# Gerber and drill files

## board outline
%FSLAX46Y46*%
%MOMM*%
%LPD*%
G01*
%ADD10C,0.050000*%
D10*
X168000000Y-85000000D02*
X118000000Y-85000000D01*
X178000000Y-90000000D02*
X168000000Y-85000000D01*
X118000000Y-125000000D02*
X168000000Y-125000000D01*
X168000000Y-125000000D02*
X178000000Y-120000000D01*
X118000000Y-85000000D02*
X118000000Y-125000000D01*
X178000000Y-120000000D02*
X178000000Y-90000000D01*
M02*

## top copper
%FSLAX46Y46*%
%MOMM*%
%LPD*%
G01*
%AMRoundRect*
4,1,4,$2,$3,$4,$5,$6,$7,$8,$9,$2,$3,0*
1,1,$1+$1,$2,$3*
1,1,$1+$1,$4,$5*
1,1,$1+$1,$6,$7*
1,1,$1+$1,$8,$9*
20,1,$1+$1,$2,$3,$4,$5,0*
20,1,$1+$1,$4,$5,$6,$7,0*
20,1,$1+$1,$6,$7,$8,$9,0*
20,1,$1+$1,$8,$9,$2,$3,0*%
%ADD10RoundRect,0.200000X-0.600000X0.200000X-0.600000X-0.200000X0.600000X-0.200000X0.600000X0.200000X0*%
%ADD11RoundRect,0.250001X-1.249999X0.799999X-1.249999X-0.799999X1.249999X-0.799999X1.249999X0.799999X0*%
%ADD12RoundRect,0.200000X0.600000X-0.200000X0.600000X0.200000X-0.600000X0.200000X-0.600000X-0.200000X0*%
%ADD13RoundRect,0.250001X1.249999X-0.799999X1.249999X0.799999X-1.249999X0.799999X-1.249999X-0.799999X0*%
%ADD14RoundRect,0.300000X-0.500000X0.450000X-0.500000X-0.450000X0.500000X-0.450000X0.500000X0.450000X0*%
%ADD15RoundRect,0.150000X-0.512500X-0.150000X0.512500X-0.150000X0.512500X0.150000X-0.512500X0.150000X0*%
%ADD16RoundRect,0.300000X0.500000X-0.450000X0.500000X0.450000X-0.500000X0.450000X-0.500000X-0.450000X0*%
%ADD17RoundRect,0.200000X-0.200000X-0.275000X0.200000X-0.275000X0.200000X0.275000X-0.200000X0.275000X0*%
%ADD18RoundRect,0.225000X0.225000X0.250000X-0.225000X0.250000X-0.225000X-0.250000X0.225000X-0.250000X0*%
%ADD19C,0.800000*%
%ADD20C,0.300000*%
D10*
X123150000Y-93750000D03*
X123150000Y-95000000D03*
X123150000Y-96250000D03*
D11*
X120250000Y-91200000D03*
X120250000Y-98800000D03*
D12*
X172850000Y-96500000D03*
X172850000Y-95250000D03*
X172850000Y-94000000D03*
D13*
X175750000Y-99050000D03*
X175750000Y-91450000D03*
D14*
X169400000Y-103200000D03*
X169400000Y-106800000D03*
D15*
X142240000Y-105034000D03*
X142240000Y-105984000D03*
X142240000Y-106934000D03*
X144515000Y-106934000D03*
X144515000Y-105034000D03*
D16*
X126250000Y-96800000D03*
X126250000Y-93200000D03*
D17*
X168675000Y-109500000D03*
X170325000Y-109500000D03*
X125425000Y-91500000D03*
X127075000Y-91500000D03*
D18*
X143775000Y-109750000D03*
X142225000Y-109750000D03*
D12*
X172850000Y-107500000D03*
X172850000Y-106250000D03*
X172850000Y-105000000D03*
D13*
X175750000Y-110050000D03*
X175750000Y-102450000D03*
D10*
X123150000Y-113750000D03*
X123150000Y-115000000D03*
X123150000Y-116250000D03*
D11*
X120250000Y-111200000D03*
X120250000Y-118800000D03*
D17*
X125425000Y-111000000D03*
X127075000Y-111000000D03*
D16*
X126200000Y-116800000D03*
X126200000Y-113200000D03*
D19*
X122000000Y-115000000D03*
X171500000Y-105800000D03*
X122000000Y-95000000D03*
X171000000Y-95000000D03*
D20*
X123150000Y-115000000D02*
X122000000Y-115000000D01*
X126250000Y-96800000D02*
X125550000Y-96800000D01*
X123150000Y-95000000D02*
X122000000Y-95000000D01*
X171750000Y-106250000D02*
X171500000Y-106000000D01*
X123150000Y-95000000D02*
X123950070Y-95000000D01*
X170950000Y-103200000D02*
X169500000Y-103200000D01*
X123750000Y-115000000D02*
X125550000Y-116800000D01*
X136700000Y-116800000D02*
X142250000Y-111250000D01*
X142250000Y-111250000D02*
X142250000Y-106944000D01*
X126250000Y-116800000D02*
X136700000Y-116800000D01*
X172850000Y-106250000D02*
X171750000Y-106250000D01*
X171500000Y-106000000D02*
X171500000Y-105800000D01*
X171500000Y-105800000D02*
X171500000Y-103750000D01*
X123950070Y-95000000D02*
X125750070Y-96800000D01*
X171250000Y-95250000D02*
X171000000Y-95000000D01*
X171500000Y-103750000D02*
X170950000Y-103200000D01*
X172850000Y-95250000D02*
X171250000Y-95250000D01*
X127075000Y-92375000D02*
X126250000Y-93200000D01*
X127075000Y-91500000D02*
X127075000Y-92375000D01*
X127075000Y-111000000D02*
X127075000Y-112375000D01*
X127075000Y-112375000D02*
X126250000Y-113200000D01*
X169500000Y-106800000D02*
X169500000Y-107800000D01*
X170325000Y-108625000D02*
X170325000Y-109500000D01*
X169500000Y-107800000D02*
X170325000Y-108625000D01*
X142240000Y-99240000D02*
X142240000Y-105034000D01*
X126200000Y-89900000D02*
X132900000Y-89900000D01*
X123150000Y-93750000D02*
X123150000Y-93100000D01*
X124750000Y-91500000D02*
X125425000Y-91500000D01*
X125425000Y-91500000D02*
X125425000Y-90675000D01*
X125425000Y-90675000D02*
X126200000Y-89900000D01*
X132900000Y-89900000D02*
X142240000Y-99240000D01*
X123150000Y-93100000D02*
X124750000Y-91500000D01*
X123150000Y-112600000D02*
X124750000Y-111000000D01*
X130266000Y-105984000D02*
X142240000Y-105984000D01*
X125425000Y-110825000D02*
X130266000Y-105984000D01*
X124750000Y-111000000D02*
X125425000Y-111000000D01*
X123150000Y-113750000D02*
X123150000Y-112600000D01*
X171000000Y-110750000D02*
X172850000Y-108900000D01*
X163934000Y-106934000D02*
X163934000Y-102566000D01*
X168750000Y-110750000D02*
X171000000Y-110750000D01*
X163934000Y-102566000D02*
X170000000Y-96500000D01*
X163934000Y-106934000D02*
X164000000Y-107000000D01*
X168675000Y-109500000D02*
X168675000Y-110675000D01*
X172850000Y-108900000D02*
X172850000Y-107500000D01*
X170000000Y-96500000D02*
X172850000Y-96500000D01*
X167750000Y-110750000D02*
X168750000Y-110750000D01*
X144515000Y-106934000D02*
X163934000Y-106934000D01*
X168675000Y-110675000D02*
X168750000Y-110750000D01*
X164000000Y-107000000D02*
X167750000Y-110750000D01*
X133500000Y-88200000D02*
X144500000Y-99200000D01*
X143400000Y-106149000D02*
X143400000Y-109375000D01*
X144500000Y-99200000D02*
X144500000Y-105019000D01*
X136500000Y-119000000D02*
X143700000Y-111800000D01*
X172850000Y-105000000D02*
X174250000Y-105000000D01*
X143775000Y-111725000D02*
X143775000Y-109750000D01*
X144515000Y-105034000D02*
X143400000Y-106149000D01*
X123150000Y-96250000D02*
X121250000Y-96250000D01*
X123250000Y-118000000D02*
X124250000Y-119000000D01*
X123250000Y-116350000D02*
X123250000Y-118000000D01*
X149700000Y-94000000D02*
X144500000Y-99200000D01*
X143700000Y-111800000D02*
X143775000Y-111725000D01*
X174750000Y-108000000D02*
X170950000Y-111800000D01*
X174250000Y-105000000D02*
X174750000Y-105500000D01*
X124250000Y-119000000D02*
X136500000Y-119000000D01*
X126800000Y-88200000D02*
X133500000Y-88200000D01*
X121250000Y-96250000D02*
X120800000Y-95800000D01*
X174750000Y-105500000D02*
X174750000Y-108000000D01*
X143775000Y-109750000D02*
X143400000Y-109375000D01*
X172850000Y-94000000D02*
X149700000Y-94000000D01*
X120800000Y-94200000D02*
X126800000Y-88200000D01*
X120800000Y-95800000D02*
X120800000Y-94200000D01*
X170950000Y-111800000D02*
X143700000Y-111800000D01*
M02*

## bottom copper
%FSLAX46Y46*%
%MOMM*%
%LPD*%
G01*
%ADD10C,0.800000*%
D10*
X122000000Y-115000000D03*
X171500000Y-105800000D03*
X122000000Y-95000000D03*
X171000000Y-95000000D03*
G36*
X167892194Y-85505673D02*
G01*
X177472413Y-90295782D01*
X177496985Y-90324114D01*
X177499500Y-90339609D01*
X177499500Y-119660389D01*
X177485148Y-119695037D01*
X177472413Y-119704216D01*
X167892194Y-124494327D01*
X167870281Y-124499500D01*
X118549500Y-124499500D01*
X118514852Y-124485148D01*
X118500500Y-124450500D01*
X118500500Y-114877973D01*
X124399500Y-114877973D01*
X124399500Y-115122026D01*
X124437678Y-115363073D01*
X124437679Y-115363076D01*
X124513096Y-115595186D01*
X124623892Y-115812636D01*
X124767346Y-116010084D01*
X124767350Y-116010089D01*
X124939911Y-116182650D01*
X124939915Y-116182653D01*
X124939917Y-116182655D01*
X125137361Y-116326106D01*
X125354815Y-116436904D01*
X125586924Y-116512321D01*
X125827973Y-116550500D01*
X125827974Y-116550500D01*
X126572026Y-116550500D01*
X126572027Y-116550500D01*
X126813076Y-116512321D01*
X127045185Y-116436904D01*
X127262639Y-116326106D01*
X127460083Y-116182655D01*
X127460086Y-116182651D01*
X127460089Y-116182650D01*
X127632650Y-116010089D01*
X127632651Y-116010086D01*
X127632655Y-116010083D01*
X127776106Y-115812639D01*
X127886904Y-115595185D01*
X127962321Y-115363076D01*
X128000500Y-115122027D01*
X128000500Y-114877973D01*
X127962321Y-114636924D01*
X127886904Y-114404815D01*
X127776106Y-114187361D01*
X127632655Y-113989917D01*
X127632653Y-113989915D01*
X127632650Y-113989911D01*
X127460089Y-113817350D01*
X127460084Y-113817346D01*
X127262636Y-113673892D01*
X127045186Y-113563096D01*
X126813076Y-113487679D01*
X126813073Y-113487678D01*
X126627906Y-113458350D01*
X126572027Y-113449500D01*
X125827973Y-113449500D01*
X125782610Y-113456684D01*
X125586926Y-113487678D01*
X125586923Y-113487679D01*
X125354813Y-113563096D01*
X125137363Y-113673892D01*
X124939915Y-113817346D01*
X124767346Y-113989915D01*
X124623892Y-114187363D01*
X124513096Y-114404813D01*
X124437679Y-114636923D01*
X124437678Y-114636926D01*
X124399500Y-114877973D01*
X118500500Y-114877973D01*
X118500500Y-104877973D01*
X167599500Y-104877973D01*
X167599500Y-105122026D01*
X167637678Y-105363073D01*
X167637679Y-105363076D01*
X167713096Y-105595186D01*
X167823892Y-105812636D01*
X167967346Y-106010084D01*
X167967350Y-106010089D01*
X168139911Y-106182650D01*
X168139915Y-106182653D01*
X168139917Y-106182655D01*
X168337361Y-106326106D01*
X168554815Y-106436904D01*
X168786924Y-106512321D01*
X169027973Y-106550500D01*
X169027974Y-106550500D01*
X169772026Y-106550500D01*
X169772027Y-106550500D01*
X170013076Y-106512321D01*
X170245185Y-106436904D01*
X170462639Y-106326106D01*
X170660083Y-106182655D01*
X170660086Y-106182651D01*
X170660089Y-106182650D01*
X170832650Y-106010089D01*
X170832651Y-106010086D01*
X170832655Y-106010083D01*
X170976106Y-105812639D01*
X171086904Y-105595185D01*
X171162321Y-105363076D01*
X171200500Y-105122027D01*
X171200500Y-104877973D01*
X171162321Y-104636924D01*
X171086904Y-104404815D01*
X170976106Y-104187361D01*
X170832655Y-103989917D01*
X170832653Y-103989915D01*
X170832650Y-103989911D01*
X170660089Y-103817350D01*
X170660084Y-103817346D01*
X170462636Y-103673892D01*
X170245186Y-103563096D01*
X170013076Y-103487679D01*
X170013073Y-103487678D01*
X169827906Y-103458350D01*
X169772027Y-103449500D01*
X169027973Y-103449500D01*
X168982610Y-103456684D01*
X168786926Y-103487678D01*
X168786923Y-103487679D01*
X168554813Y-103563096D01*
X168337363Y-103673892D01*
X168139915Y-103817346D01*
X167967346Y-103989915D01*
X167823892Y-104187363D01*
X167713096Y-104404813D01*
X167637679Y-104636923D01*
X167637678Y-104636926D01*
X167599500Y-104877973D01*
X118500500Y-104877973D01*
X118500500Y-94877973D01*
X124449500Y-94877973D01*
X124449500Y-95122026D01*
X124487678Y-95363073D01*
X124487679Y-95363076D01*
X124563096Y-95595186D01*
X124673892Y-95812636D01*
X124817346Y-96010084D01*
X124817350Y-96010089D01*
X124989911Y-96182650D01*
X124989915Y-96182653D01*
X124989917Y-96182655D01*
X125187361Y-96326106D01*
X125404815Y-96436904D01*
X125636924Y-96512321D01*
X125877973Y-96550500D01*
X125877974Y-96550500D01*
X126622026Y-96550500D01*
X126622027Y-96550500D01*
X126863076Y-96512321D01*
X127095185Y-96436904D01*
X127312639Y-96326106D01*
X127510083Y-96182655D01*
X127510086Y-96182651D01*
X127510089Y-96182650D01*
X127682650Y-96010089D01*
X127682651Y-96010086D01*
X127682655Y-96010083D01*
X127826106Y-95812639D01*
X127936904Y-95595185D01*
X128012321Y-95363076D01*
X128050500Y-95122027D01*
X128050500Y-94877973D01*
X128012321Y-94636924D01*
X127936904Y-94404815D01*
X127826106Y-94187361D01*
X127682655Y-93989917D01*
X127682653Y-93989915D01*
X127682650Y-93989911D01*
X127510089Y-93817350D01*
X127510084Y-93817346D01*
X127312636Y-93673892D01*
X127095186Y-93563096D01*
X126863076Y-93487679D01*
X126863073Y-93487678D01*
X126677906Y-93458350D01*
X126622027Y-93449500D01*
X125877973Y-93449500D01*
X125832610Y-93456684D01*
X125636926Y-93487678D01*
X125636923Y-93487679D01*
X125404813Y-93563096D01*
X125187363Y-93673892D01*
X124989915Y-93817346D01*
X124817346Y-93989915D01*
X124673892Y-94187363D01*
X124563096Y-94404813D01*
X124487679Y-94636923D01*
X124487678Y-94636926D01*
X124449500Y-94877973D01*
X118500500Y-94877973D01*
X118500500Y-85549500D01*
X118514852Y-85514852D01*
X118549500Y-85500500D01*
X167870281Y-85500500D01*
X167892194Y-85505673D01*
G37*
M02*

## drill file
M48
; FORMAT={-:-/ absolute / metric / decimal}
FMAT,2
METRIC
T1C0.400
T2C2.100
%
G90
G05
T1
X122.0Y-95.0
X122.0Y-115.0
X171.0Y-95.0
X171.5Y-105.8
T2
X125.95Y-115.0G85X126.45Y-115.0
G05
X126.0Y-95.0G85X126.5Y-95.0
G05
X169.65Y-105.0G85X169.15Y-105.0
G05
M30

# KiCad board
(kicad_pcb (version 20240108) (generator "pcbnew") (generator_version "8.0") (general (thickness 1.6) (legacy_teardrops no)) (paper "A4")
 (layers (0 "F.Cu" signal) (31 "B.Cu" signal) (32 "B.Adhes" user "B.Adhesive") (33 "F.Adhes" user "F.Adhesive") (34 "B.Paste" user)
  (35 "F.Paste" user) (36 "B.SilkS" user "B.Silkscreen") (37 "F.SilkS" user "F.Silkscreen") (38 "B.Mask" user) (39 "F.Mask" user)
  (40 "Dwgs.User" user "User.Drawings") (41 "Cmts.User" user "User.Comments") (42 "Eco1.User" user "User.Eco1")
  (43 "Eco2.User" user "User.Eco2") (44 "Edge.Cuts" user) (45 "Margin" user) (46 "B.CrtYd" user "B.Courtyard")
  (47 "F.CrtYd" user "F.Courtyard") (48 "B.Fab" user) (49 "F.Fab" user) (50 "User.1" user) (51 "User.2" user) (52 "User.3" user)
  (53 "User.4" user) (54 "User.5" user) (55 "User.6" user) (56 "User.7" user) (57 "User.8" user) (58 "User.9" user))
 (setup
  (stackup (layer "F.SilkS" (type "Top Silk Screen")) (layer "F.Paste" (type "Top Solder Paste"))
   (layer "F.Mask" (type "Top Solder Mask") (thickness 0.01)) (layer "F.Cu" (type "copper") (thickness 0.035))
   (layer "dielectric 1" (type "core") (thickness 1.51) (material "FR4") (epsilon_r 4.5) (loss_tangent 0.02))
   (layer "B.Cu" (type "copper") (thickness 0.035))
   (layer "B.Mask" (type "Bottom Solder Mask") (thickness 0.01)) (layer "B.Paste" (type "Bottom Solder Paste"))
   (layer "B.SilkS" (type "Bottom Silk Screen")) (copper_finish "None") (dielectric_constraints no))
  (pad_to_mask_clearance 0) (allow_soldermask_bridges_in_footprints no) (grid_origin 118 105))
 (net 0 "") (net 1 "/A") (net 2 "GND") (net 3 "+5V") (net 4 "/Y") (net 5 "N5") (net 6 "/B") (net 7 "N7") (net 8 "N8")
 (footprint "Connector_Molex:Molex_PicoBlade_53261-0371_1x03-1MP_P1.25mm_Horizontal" (layer "F.Cu") (at 120.75 95 -90)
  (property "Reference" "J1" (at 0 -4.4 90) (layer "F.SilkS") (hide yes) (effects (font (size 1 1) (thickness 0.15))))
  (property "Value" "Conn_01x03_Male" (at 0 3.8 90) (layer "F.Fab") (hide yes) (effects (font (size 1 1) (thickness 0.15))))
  (pad "1" smd roundrect (at -1.25 -2.4 270) (size 0.8 1.6) (layers "F.Cu" "F.Paste" "F.Mask") (roundrect_rratio 0.25) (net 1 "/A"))
  (pad "2" smd roundrect (at 0 -2.4 270) (size 0.8 1.6) (layers "F.Cu" "F.Paste" "F.Mask") (roundrect_rratio 0.25) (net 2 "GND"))
  (pad "3" smd roundrect (at 1.25 -2.4 270) (size 0.8 1.6) (layers "F.Cu" "F.Paste" "F.Mask") (roundrect_rratio 0.25) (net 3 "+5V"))
  (pad "MP" smd roundrect (at -3.8 0.5 270) (size 2.1 3) (layers "F.Cu" "F.Paste" "F.Mask") (roundrect_rratio 0.1190480952))
  (pad "MP" smd roundrect (at 3.8 0.5 270) (size 2.1 3) (layers "F.Cu" "F.Paste" "F.Mask") (roundrect_rratio 0.1190480952)))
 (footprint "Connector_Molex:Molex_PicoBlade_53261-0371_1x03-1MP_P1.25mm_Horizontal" (layer "F.Cu") (at 175.25 95.25 90)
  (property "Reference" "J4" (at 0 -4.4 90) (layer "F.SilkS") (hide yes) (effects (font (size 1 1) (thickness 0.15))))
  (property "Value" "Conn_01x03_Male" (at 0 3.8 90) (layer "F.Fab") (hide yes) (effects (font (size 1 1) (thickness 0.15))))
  (pad "1" smd roundrect (at -1.25 -2.4 90) (size 0.8 1.6) (layers "F.Cu" "F.Paste" "F.Mask") (roundrect_rratio 0.25) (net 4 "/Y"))
  (pad "2" smd roundrect (at 0 -2.4 90) (size 0.8 1.6) (layers "F.Cu" "F.Paste" "F.Mask") (roundrect_rratio 0.25) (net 2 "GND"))
  (pad "3" smd roundrect (at 1.25 -2.4 90) (size 0.8 1.6) (layers "F.Cu" "F.Paste" "F.Mask") (roundrect_rratio 0.25) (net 3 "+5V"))
  (pad "MP" smd roundrect (at -3.8 0.5 90) (size 2.1 3) (layers "F.Cu" "F.Paste" "F.Mask") (roundrect_rratio 0.1190480952))
  (pad "MP" smd roundrect (at 3.8 0.5 90) (size 2.1 3) (layers "F.Cu" "F.Paste" "F.Mask") (roundrect_rratio 0.1190480952)))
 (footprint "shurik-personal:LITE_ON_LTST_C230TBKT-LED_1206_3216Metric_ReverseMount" (layer "F.Cu") (at 169.4 105 -90)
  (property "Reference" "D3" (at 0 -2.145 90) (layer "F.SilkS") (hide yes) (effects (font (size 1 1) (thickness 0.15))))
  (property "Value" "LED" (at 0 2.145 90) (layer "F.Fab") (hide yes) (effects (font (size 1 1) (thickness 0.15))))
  (pad "" np_thru_hole oval (at 0 0 270) (size 2.1 2.6) (drill oval 2.1 2.6) (layers "F&B.Cu" "*.Mask"))
  (pad "1" smd roundrect (at -1.8 0 270) (size 1.5 1.6) (layers "F.Cu" "F.Paste" "F.Mask") (roundrect_rratio 0.2) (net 2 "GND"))
  (pad "2" smd roundrect (at 1.8 0 270) (size 1.5 1.6) (layers "F.Cu" "F.Paste" "F.Mask") (roundrect_rratio 0.2) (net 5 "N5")))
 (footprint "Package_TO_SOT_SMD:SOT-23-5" (layer "F.Cu") (at 143.3775 105.984)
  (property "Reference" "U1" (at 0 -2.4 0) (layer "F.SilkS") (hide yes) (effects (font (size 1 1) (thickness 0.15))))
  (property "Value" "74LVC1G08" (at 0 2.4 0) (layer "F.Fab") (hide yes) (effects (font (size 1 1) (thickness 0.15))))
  (pad "1" smd roundrect (at -1.1375 -0.95) (size 1.325 0.6) (layers "F.Cu" "F.Paste" "F.Mask") (roundrect_rratio 0.25) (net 1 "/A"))
  (pad "2" smd roundrect (at -1.1375 0) (size 1.325 0.6) (layers "F.Cu" "F.Paste" "F.Mask") (roundrect_rratio 0.25) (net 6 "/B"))
  (pad "3" smd roundrect (at -1.1375 0.95) (size 1.325 0.6) (layers "F.Cu" "F.Paste" "F.Mask") (roundrect_rratio 0.25) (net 2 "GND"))
  (pad "4" smd roundrect (at 1.1375 0.95) (size 1.325 0.6) (layers "F.Cu" "F.Paste" "F.Mask") (roundrect_rratio 0.25) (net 4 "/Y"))
  (pad "5" smd roundrect (at 1.1375 -0.95) (size 1.325 0.6) (layers "F.Cu" "F.Paste" "F.Mask") (roundrect_rratio 0.25) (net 3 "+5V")))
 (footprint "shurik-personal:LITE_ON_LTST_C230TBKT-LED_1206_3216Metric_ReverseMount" (layer "F.Cu") (at 126.25 95 90)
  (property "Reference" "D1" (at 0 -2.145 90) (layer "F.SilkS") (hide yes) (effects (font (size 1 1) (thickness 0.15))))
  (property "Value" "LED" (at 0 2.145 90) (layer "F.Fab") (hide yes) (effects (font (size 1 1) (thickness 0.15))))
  (pad "" np_thru_hole oval (at 0 0 90) (size 2.1 2.6) (drill oval 2.1 2.6) (layers "F&B.Cu" "*.Mask"))
  (pad "1" smd roundrect (at -1.8 0 90) (size 1.5 1.6) (layers "F.Cu" "F.Paste" "F.Mask") (roundrect_rratio 0.2) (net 2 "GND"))
  (pad "2" smd roundrect (at 1.8 0 90) (size 1.5 1.6) (layers "F.Cu" "F.Paste" "F.Mask") (roundrect_rratio 0.2) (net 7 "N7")))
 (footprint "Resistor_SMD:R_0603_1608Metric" (layer "F.Cu") (at 169.5 109.5)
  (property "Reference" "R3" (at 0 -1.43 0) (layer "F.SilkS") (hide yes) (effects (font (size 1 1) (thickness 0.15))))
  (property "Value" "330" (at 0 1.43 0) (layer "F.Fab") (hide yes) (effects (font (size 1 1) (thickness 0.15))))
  (pad "1" smd roundrect (at -0.825 0) (size 0.8 0.95) (layers "F.Cu" "F.Paste" "F.Mask") (roundrect_rratio 0.25) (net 4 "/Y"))
  (pad "2" smd roundrect (at 0.825 0) (size 0.8 0.95) (layers "F.Cu" "F.Paste" "F.Mask") (roundrect_rratio 0.25) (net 5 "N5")))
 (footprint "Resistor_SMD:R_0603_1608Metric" (layer "F.Cu") (at 126.25 91.5)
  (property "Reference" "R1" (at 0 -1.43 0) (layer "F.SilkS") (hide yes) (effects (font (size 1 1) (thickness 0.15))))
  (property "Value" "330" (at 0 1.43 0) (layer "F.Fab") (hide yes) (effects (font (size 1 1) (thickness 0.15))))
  (pad "1" smd roundrect (at -0.825 0) (size 0.8 0.95) (layers "F.Cu" "F.Paste" "F.Mask") (roundrect_rratio 0.25) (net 1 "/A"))
  (pad "2" smd roundrect (at 0.825 0) (size 0.8 0.95) (layers "F.Cu" "F.Paste" "F.Mask") (roundrect_rratio 0.25) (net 7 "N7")))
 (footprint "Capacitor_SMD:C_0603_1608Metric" (layer "F.Cu") (at 143 109.75 180)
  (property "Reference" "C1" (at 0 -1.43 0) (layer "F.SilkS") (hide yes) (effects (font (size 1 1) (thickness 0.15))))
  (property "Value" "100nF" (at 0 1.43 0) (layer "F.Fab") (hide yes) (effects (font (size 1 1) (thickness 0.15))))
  (pad "1" smd roundrect (at -0.775 0 180) (size 0.9 0.95) (layers "F.Cu" "F.Paste" "F.Mask") (roundrect_rratio 0.25) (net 3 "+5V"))
  (pad "2" smd roundrect (at 0.775 0 180) (size 0.9 0.95) (layers "F.Cu" "F.Paste" "F.Mask") (roundrect_rratio 0.25) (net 2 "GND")))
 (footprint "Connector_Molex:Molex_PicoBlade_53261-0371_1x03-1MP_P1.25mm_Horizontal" (layer "F.Cu") (at 175.25 106.25 90)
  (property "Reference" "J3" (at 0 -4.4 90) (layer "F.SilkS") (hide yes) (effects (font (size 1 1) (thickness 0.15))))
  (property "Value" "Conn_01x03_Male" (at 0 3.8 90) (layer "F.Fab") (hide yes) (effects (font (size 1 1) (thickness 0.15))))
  (pad "1" smd roundrect (at -1.25 -2.4 90) (size 0.8 1.6) (layers "F.Cu" "F.Paste" "F.Mask") (roundrect_rratio 0.25) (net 4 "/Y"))
  (pad "2" smd roundrect (at 0 -2.4 90) (size 0.8 1.6) (layers "F.Cu" "F.Paste" "F.Mask") (roundrect_rratio 0.25) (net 2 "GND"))
  (pad "3" smd roundrect (at 1.25 -2.4 90) (size 0.8 1.6) (layers "F.Cu" "F.Paste" "F.Mask") (roundrect_rratio 0.25) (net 3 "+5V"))
  (pad "MP" smd roundrect (at -3.8 0.5 90) (size 2.1 3) (layers "F.Cu" "F.Paste" "F.Mask") (roundrect_rratio 0.1190480952))
  (pad "MP" smd roundrect (at 3.8 0.5 90) (size 2.1 3) (layers "F.Cu" "F.Paste" "F.Mask") (roundrect_rratio 0.1190480952)))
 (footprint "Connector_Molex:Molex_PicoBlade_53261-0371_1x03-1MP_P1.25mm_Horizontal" (layer "F.Cu") (at 120.75 115 -90)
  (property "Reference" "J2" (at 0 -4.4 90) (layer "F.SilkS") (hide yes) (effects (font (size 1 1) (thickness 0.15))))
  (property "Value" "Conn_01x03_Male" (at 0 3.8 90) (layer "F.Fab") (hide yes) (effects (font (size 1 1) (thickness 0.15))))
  (pad "1" smd roundrect (at -1.25 -2.4 270) (size 0.8 1.6) (layers "F.Cu" "F.Paste" "F.Mask") (roundrect_rratio 0.25) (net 6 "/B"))
  (pad "2" smd roundrect (at 0 -2.4 270) (size 0.8 1.6) (layers "F.Cu" "F.Paste" "F.Mask") (roundrect_rratio 0.25) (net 2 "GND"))
  (pad "3" smd roundrect (at 1.25 -2.4 270) (size 0.8 1.6) (layers "F.Cu" "F.Paste" "F.Mask") (roundrect_rratio 0.25) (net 3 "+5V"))
  (pad "MP" smd roundrect (at -3.8 0.5 270) (size 2.1 3) (layers "F.Cu" "F.Paste" "F.Mask") (roundrect_rratio 0.1190480952))
  (pad "MP" smd roundrect (at 3.8 0.5 270) (size 2.1 3) (layers "F.Cu" "F.Paste" "F.Mask") (roundrect_rratio 0.1190480952)))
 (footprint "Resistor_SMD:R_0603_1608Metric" (layer "F.Cu") (at 126.25 111)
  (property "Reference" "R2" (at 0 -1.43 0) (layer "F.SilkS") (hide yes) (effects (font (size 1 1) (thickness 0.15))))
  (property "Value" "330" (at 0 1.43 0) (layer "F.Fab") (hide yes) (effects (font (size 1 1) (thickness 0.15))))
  (pad "1" smd roundrect (at -0.825 0) (size 0.8 0.95) (layers "F.Cu" "F.Paste" "F.Mask") (roundrect_rratio 0.25) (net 6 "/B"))
  (pad "2" smd roundrect (at 0.825 0) (size 0.8 0.95) (layers "F.Cu" "F.Paste" "F.Mask") (roundrect_rratio 0.25) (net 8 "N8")))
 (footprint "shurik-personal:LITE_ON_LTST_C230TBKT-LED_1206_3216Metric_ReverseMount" (layer "F.Cu") (at 126.2 115 90)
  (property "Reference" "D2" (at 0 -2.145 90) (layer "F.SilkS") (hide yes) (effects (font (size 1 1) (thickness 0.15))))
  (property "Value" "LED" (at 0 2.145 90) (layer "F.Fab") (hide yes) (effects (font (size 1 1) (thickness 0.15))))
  (pad "" np_thru_hole oval (at 0 0 90) (size 2.1 2.6) (drill oval 2.1 2.6) (layers "F&B.Cu" "*.Mask"))
  (pad "1" smd roundrect (at -1.8 0 90) (size 1.5 1.6) (layers "F.Cu" "F.Paste" "F.Mask") (roundrect_rratio 0.2) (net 2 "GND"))
  (pad "2" smd roundrect (at 1.8 0 90) (size 1.5 1.6) (layers "F.Cu" "F.Paste" "F.Mask") (roundrect_rratio 0.2) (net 8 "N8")))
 (gr_line (start 168 85) (end 118 85) (stroke (width 0.05) (type solid)) (layer "Edge.Cuts"))
 (gr_line (start 178 90) (end 168 85) (stroke (width 0.05) (type solid)) (layer "Edge.Cuts"))
 (gr_line (start 118 125) (end 168 125) (stroke (width 0.05) (type solid)) (layer "Edge.Cuts"))
 (gr_line (start 168 125) (end 178 120) (stroke (width 0.05) (type solid)) (layer "Edge.Cuts"))
 (gr_line (start 118 85) (end 118 125) (stroke (width 0.05) (type solid)) (layer "Edge.Cuts"))
 (gr_line (start 178 120) (end 178 90) (stroke (width 0.05) (type solid)) (layer "Edge.Cuts"))
 (segment (start 123.15 115) (end 122 115) (width 0.3) (layer "F.Cu") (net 2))
 (segment (start 126.25 96.8) (end 125.55 96.8) (width 0.3) (layer "F.Cu") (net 2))
 (segment (start 123.15 95) (end 122 95) (width 0.3) (layer "F.Cu") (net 2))
 (segment (start 171.75 106.25) (end 171.5 106) (width 0.3) (layer "F.Cu") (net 2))
 (segment (start 123.15 95) (end 123.95007 95) (width 0.3) (layer "F.Cu") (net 2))
 (segment (start 170.95 103.2) (end 169.5 103.2) (width 0.3) (layer "F.Cu") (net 2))
 (segment (start 123.75 115) (end 125.55 116.8) (width 0.3) (layer "F.Cu") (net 2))
 (segment (start 136.7 116.8) (end 142.25 111.25) (width 0.3) (layer "F.Cu") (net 2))
 (segment (start 142.25 111.25) (end 142.25 106.944) (width 0.3) (layer "F.Cu") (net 2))
 (segment (start 126.25 116.8) (end 136.7 116.8) (width 0.3) (layer "F.Cu") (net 2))
 (segment (start 172.85 106.25) (end 171.75 106.25) (width 0.3) (layer "F.Cu") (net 2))
 (segment (start 171.5 106) (end 171.5 105.8) (width 0.3) (layer "F.Cu") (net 2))
 (segment (start 171.5 105.8) (end 171.5 103.75) (width 0.3) (layer "F.Cu") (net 2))
 (segment (start 123.95007 95) (end 125.75007 96.8) (width 0.3) (layer "F.Cu") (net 2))
 (segment (start 171.25 95.25) (end 171 95) (width 0.3) (layer "F.Cu") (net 2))
 (segment (start 171.5 103.75) (end 170.95 103.2) (width 0.3) (layer "F.Cu") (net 2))
 (segment (start 172.85 95.25) (end 171.25 95.25) (width 0.3) (layer "F.Cu") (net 2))
 (via (at 122 115) (size 0.8) (drill 0.4) (layers "F.Cu" "B.Cu") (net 2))
 (via (at 171.5 105.8) (size 0.8) (drill 0.4) (layers "F.Cu" "B.Cu") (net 2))
 (via (at 122 95) (size 0.8) (drill 0.4) (layers "F.Cu" "B.Cu") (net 2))
 (via (at 171 95) (size 0.8) (drill 0.4) (layers "F.Cu" "B.Cu") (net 2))
 (segment (start 127.075 92.375) (end 126.25 93.2) (width 0.3) (layer "F.Cu") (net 7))
 (segment (start 127.075 91.5) (end 127.075 92.375) (width 0.3) (layer "F.Cu") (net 7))
 (segment (start 127.075 111) (end 127.075 112.375) (width 0.3) (layer "F.Cu") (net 8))
 (segment (start 127.075 112.375) (end 126.25 113.2) (width 0.3) (layer "F.Cu") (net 8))
 (segment (start 169.5 106.8) (end 169.5 107.8) (width 0.3) (layer "F.Cu") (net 5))
 (segment (start 170.325 108.625) (end 170.325 109.5) (width 0.3) (layer "F.Cu") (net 5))
 (segment (start 169.5 107.8) (end 170.325 108.625) (width 0.3) (layer "F.Cu") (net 5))
 (segment (start 142.24 99.24) (end 142.24 105.034) (width 0.3) (layer "F.Cu") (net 1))
 (segment (start 126.2 89.9) (end 132.9 89.9) (width 0.3) (layer "F.Cu") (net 1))
 (segment (start 123.15 93.75) (end 123.15 93.1) (width 0.3) (layer "F.Cu") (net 1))
 (segment (start 124.75 91.5) (end 125.425 91.5) (width 0.3) (layer "F.Cu") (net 1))
 (segment (start 125.425 91.5) (end 125.425 90.675) (width 0.3) (layer "F.Cu") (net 1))
 (segment (start 125.425 90.675) (end 126.2 89.9) (width 0.3) (layer "F.Cu") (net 1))
 (segment (start 132.9 89.9) (end 142.24 99.24) (width 0.3) (layer "F.Cu") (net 1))
 (segment (start 123.15 93.1) (end 124.75 91.5) (width 0.3) (layer "F.Cu") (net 1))
 (segment (start 123.15 112.6) (end 124.75 111) (width 0.3) (layer "F.Cu") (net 6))
 (segment (start 130.266 105.984) (end 142.24 105.984) (width 0.3) (layer "F.Cu") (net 6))
 (segment (start 125.425 110.825) (end 130.266 105.984) (width 0.3) (layer "F.Cu") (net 6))
 (segment (start 124.75 111) (end 125.425 111) (width 0.3) (layer "F.Cu") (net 6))
 (segment (start 123.15 113.75) (end 123.15 112.6) (width 0.3) (layer "F.Cu") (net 6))
 (segment (start 171 110.75) (end 172.85 108.9) (width 0.3) (layer "F.Cu") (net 4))
 (segment (start 163.934 106.934) (end 163.934 102.566) (width 0.3) (layer "F.Cu") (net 4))
 (segment (start 168.75 110.75) (end 171 110.75) (width 0.3) (layer "F.Cu") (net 4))
 (segment (start 163.934 102.566) (end 170 96.5) (width 0.3) (layer "F.Cu") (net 4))
 (segment (start 163.934 106.934) (end 164 107) (width 0.3) (layer "F.Cu") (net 4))
 (segment (start 168.675 109.5) (end 168.675 110.675) (width 0.3) (layer "F.Cu") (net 4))
 (segment (start 172.85 108.9) (end 172.85 107.5) (width 0.3) (layer "F.Cu") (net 4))
 (segment (start 170 96.5) (end 172.85 96.5) (width 0.3) (layer "F.Cu") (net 4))
 (segment (start 167.75 110.75) (end 168.75 110.75) (width 0.3) (layer "F.Cu") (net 4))
 (segment (start 144.515 106.934) (end 163.934 106.934) (width 0.3) (layer "F.Cu") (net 4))
 (segment (start 168.675 110.675) (end 168.75 110.75) (width 0.3) (layer "F.Cu") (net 4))
 (segment (start 164 107) (end 167.75 110.75) (width 0.3) (layer "F.Cu") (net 4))
 (segment (start 133.5 88.2) (end 144.5 99.2) (width 0.3) (layer "F.Cu") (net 3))
 (segment (start 143.4 106.149) (end 143.4 109.375) (width 0.3) (layer "F.Cu") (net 3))
 (segment (start 144.5 99.2) (end 144.5 105.019) (width 0.3) (layer "F.Cu") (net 3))
 (segment (start 136.5 119) (end 143.7 111.8) (width 0.3) (layer "F.Cu") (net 3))
 (segment (start 172.85 105) (end 174.25 105) (width 0.3) (layer "F.Cu") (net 3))
 (segment (start 143.775 111.725) (end 143.775 109.75) (width 0.3) (layer "F.Cu") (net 3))
 (segment (start 144.515 105.034) (end 143.4 106.149) (width 0.3) (layer "F.Cu") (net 3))
 (segment (start 123.15 96.25) (end 121.25 96.25) (width 0.3) (layer "F.Cu") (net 3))
 (segment (start 123.25 118) (end 124.25 119) (width 0.3) (layer "F.Cu") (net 3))
 (segment (start 123.25 116.35) (end 123.25 118) (width 0.3) (layer "F.Cu") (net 3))
 (segment (start 149.7 94) (end 144.5 99.2) (width 0.3) (layer "F.Cu") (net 3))
 (segment (start 143.7 111.8) (end 143.775 111.725) (width 0.3) (layer "F.Cu") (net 3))
 (segment (start 174.75 108) (end 170.95 111.8) (width 0.3) (layer "F.Cu") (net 3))
 (segment (start 174.25 105) (end 174.75 105.5) (width 0.3) (layer "F.Cu") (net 3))
 (segment (start 124.25 119) (end 136.5 119) (width 0.3) (layer "F.Cu") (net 3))
 (segment (start 126.8 88.2) (end 133.5 88.2) (width 0.3) (layer "F.Cu") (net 3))
 (segment (start 121.25 96.25) (end 120.8 95.8) (width 0.3) (layer "F.Cu") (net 3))
 (segment (start 174.75 105.5) (end 174.75 108) (width 0.3) (layer "F.Cu") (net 3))
 (segment (start 143.775 109.75) (end 143.4 109.375) (width 0.3) (layer "F.Cu") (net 3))
 (segment (start 172.85 94) (end 149.7 94) (width 0.3) (layer "F.Cu") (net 3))
 (segment (start 120.8 94.2) (end 126.8 88.2) (width 0.3) (layer "F.Cu") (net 3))
 (segment (start 120.8 95.8) (end 120.8 94.2) (width 0.3) (layer "F.Cu") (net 3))
 (segment (start 170.95 111.8) (end 143.7 111.8) (width 0.3) (layer "F.Cu") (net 3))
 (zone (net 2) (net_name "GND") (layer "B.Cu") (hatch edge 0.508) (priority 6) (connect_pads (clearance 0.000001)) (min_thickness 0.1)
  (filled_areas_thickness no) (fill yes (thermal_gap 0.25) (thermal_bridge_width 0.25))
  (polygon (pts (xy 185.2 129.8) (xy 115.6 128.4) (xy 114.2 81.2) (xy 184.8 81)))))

